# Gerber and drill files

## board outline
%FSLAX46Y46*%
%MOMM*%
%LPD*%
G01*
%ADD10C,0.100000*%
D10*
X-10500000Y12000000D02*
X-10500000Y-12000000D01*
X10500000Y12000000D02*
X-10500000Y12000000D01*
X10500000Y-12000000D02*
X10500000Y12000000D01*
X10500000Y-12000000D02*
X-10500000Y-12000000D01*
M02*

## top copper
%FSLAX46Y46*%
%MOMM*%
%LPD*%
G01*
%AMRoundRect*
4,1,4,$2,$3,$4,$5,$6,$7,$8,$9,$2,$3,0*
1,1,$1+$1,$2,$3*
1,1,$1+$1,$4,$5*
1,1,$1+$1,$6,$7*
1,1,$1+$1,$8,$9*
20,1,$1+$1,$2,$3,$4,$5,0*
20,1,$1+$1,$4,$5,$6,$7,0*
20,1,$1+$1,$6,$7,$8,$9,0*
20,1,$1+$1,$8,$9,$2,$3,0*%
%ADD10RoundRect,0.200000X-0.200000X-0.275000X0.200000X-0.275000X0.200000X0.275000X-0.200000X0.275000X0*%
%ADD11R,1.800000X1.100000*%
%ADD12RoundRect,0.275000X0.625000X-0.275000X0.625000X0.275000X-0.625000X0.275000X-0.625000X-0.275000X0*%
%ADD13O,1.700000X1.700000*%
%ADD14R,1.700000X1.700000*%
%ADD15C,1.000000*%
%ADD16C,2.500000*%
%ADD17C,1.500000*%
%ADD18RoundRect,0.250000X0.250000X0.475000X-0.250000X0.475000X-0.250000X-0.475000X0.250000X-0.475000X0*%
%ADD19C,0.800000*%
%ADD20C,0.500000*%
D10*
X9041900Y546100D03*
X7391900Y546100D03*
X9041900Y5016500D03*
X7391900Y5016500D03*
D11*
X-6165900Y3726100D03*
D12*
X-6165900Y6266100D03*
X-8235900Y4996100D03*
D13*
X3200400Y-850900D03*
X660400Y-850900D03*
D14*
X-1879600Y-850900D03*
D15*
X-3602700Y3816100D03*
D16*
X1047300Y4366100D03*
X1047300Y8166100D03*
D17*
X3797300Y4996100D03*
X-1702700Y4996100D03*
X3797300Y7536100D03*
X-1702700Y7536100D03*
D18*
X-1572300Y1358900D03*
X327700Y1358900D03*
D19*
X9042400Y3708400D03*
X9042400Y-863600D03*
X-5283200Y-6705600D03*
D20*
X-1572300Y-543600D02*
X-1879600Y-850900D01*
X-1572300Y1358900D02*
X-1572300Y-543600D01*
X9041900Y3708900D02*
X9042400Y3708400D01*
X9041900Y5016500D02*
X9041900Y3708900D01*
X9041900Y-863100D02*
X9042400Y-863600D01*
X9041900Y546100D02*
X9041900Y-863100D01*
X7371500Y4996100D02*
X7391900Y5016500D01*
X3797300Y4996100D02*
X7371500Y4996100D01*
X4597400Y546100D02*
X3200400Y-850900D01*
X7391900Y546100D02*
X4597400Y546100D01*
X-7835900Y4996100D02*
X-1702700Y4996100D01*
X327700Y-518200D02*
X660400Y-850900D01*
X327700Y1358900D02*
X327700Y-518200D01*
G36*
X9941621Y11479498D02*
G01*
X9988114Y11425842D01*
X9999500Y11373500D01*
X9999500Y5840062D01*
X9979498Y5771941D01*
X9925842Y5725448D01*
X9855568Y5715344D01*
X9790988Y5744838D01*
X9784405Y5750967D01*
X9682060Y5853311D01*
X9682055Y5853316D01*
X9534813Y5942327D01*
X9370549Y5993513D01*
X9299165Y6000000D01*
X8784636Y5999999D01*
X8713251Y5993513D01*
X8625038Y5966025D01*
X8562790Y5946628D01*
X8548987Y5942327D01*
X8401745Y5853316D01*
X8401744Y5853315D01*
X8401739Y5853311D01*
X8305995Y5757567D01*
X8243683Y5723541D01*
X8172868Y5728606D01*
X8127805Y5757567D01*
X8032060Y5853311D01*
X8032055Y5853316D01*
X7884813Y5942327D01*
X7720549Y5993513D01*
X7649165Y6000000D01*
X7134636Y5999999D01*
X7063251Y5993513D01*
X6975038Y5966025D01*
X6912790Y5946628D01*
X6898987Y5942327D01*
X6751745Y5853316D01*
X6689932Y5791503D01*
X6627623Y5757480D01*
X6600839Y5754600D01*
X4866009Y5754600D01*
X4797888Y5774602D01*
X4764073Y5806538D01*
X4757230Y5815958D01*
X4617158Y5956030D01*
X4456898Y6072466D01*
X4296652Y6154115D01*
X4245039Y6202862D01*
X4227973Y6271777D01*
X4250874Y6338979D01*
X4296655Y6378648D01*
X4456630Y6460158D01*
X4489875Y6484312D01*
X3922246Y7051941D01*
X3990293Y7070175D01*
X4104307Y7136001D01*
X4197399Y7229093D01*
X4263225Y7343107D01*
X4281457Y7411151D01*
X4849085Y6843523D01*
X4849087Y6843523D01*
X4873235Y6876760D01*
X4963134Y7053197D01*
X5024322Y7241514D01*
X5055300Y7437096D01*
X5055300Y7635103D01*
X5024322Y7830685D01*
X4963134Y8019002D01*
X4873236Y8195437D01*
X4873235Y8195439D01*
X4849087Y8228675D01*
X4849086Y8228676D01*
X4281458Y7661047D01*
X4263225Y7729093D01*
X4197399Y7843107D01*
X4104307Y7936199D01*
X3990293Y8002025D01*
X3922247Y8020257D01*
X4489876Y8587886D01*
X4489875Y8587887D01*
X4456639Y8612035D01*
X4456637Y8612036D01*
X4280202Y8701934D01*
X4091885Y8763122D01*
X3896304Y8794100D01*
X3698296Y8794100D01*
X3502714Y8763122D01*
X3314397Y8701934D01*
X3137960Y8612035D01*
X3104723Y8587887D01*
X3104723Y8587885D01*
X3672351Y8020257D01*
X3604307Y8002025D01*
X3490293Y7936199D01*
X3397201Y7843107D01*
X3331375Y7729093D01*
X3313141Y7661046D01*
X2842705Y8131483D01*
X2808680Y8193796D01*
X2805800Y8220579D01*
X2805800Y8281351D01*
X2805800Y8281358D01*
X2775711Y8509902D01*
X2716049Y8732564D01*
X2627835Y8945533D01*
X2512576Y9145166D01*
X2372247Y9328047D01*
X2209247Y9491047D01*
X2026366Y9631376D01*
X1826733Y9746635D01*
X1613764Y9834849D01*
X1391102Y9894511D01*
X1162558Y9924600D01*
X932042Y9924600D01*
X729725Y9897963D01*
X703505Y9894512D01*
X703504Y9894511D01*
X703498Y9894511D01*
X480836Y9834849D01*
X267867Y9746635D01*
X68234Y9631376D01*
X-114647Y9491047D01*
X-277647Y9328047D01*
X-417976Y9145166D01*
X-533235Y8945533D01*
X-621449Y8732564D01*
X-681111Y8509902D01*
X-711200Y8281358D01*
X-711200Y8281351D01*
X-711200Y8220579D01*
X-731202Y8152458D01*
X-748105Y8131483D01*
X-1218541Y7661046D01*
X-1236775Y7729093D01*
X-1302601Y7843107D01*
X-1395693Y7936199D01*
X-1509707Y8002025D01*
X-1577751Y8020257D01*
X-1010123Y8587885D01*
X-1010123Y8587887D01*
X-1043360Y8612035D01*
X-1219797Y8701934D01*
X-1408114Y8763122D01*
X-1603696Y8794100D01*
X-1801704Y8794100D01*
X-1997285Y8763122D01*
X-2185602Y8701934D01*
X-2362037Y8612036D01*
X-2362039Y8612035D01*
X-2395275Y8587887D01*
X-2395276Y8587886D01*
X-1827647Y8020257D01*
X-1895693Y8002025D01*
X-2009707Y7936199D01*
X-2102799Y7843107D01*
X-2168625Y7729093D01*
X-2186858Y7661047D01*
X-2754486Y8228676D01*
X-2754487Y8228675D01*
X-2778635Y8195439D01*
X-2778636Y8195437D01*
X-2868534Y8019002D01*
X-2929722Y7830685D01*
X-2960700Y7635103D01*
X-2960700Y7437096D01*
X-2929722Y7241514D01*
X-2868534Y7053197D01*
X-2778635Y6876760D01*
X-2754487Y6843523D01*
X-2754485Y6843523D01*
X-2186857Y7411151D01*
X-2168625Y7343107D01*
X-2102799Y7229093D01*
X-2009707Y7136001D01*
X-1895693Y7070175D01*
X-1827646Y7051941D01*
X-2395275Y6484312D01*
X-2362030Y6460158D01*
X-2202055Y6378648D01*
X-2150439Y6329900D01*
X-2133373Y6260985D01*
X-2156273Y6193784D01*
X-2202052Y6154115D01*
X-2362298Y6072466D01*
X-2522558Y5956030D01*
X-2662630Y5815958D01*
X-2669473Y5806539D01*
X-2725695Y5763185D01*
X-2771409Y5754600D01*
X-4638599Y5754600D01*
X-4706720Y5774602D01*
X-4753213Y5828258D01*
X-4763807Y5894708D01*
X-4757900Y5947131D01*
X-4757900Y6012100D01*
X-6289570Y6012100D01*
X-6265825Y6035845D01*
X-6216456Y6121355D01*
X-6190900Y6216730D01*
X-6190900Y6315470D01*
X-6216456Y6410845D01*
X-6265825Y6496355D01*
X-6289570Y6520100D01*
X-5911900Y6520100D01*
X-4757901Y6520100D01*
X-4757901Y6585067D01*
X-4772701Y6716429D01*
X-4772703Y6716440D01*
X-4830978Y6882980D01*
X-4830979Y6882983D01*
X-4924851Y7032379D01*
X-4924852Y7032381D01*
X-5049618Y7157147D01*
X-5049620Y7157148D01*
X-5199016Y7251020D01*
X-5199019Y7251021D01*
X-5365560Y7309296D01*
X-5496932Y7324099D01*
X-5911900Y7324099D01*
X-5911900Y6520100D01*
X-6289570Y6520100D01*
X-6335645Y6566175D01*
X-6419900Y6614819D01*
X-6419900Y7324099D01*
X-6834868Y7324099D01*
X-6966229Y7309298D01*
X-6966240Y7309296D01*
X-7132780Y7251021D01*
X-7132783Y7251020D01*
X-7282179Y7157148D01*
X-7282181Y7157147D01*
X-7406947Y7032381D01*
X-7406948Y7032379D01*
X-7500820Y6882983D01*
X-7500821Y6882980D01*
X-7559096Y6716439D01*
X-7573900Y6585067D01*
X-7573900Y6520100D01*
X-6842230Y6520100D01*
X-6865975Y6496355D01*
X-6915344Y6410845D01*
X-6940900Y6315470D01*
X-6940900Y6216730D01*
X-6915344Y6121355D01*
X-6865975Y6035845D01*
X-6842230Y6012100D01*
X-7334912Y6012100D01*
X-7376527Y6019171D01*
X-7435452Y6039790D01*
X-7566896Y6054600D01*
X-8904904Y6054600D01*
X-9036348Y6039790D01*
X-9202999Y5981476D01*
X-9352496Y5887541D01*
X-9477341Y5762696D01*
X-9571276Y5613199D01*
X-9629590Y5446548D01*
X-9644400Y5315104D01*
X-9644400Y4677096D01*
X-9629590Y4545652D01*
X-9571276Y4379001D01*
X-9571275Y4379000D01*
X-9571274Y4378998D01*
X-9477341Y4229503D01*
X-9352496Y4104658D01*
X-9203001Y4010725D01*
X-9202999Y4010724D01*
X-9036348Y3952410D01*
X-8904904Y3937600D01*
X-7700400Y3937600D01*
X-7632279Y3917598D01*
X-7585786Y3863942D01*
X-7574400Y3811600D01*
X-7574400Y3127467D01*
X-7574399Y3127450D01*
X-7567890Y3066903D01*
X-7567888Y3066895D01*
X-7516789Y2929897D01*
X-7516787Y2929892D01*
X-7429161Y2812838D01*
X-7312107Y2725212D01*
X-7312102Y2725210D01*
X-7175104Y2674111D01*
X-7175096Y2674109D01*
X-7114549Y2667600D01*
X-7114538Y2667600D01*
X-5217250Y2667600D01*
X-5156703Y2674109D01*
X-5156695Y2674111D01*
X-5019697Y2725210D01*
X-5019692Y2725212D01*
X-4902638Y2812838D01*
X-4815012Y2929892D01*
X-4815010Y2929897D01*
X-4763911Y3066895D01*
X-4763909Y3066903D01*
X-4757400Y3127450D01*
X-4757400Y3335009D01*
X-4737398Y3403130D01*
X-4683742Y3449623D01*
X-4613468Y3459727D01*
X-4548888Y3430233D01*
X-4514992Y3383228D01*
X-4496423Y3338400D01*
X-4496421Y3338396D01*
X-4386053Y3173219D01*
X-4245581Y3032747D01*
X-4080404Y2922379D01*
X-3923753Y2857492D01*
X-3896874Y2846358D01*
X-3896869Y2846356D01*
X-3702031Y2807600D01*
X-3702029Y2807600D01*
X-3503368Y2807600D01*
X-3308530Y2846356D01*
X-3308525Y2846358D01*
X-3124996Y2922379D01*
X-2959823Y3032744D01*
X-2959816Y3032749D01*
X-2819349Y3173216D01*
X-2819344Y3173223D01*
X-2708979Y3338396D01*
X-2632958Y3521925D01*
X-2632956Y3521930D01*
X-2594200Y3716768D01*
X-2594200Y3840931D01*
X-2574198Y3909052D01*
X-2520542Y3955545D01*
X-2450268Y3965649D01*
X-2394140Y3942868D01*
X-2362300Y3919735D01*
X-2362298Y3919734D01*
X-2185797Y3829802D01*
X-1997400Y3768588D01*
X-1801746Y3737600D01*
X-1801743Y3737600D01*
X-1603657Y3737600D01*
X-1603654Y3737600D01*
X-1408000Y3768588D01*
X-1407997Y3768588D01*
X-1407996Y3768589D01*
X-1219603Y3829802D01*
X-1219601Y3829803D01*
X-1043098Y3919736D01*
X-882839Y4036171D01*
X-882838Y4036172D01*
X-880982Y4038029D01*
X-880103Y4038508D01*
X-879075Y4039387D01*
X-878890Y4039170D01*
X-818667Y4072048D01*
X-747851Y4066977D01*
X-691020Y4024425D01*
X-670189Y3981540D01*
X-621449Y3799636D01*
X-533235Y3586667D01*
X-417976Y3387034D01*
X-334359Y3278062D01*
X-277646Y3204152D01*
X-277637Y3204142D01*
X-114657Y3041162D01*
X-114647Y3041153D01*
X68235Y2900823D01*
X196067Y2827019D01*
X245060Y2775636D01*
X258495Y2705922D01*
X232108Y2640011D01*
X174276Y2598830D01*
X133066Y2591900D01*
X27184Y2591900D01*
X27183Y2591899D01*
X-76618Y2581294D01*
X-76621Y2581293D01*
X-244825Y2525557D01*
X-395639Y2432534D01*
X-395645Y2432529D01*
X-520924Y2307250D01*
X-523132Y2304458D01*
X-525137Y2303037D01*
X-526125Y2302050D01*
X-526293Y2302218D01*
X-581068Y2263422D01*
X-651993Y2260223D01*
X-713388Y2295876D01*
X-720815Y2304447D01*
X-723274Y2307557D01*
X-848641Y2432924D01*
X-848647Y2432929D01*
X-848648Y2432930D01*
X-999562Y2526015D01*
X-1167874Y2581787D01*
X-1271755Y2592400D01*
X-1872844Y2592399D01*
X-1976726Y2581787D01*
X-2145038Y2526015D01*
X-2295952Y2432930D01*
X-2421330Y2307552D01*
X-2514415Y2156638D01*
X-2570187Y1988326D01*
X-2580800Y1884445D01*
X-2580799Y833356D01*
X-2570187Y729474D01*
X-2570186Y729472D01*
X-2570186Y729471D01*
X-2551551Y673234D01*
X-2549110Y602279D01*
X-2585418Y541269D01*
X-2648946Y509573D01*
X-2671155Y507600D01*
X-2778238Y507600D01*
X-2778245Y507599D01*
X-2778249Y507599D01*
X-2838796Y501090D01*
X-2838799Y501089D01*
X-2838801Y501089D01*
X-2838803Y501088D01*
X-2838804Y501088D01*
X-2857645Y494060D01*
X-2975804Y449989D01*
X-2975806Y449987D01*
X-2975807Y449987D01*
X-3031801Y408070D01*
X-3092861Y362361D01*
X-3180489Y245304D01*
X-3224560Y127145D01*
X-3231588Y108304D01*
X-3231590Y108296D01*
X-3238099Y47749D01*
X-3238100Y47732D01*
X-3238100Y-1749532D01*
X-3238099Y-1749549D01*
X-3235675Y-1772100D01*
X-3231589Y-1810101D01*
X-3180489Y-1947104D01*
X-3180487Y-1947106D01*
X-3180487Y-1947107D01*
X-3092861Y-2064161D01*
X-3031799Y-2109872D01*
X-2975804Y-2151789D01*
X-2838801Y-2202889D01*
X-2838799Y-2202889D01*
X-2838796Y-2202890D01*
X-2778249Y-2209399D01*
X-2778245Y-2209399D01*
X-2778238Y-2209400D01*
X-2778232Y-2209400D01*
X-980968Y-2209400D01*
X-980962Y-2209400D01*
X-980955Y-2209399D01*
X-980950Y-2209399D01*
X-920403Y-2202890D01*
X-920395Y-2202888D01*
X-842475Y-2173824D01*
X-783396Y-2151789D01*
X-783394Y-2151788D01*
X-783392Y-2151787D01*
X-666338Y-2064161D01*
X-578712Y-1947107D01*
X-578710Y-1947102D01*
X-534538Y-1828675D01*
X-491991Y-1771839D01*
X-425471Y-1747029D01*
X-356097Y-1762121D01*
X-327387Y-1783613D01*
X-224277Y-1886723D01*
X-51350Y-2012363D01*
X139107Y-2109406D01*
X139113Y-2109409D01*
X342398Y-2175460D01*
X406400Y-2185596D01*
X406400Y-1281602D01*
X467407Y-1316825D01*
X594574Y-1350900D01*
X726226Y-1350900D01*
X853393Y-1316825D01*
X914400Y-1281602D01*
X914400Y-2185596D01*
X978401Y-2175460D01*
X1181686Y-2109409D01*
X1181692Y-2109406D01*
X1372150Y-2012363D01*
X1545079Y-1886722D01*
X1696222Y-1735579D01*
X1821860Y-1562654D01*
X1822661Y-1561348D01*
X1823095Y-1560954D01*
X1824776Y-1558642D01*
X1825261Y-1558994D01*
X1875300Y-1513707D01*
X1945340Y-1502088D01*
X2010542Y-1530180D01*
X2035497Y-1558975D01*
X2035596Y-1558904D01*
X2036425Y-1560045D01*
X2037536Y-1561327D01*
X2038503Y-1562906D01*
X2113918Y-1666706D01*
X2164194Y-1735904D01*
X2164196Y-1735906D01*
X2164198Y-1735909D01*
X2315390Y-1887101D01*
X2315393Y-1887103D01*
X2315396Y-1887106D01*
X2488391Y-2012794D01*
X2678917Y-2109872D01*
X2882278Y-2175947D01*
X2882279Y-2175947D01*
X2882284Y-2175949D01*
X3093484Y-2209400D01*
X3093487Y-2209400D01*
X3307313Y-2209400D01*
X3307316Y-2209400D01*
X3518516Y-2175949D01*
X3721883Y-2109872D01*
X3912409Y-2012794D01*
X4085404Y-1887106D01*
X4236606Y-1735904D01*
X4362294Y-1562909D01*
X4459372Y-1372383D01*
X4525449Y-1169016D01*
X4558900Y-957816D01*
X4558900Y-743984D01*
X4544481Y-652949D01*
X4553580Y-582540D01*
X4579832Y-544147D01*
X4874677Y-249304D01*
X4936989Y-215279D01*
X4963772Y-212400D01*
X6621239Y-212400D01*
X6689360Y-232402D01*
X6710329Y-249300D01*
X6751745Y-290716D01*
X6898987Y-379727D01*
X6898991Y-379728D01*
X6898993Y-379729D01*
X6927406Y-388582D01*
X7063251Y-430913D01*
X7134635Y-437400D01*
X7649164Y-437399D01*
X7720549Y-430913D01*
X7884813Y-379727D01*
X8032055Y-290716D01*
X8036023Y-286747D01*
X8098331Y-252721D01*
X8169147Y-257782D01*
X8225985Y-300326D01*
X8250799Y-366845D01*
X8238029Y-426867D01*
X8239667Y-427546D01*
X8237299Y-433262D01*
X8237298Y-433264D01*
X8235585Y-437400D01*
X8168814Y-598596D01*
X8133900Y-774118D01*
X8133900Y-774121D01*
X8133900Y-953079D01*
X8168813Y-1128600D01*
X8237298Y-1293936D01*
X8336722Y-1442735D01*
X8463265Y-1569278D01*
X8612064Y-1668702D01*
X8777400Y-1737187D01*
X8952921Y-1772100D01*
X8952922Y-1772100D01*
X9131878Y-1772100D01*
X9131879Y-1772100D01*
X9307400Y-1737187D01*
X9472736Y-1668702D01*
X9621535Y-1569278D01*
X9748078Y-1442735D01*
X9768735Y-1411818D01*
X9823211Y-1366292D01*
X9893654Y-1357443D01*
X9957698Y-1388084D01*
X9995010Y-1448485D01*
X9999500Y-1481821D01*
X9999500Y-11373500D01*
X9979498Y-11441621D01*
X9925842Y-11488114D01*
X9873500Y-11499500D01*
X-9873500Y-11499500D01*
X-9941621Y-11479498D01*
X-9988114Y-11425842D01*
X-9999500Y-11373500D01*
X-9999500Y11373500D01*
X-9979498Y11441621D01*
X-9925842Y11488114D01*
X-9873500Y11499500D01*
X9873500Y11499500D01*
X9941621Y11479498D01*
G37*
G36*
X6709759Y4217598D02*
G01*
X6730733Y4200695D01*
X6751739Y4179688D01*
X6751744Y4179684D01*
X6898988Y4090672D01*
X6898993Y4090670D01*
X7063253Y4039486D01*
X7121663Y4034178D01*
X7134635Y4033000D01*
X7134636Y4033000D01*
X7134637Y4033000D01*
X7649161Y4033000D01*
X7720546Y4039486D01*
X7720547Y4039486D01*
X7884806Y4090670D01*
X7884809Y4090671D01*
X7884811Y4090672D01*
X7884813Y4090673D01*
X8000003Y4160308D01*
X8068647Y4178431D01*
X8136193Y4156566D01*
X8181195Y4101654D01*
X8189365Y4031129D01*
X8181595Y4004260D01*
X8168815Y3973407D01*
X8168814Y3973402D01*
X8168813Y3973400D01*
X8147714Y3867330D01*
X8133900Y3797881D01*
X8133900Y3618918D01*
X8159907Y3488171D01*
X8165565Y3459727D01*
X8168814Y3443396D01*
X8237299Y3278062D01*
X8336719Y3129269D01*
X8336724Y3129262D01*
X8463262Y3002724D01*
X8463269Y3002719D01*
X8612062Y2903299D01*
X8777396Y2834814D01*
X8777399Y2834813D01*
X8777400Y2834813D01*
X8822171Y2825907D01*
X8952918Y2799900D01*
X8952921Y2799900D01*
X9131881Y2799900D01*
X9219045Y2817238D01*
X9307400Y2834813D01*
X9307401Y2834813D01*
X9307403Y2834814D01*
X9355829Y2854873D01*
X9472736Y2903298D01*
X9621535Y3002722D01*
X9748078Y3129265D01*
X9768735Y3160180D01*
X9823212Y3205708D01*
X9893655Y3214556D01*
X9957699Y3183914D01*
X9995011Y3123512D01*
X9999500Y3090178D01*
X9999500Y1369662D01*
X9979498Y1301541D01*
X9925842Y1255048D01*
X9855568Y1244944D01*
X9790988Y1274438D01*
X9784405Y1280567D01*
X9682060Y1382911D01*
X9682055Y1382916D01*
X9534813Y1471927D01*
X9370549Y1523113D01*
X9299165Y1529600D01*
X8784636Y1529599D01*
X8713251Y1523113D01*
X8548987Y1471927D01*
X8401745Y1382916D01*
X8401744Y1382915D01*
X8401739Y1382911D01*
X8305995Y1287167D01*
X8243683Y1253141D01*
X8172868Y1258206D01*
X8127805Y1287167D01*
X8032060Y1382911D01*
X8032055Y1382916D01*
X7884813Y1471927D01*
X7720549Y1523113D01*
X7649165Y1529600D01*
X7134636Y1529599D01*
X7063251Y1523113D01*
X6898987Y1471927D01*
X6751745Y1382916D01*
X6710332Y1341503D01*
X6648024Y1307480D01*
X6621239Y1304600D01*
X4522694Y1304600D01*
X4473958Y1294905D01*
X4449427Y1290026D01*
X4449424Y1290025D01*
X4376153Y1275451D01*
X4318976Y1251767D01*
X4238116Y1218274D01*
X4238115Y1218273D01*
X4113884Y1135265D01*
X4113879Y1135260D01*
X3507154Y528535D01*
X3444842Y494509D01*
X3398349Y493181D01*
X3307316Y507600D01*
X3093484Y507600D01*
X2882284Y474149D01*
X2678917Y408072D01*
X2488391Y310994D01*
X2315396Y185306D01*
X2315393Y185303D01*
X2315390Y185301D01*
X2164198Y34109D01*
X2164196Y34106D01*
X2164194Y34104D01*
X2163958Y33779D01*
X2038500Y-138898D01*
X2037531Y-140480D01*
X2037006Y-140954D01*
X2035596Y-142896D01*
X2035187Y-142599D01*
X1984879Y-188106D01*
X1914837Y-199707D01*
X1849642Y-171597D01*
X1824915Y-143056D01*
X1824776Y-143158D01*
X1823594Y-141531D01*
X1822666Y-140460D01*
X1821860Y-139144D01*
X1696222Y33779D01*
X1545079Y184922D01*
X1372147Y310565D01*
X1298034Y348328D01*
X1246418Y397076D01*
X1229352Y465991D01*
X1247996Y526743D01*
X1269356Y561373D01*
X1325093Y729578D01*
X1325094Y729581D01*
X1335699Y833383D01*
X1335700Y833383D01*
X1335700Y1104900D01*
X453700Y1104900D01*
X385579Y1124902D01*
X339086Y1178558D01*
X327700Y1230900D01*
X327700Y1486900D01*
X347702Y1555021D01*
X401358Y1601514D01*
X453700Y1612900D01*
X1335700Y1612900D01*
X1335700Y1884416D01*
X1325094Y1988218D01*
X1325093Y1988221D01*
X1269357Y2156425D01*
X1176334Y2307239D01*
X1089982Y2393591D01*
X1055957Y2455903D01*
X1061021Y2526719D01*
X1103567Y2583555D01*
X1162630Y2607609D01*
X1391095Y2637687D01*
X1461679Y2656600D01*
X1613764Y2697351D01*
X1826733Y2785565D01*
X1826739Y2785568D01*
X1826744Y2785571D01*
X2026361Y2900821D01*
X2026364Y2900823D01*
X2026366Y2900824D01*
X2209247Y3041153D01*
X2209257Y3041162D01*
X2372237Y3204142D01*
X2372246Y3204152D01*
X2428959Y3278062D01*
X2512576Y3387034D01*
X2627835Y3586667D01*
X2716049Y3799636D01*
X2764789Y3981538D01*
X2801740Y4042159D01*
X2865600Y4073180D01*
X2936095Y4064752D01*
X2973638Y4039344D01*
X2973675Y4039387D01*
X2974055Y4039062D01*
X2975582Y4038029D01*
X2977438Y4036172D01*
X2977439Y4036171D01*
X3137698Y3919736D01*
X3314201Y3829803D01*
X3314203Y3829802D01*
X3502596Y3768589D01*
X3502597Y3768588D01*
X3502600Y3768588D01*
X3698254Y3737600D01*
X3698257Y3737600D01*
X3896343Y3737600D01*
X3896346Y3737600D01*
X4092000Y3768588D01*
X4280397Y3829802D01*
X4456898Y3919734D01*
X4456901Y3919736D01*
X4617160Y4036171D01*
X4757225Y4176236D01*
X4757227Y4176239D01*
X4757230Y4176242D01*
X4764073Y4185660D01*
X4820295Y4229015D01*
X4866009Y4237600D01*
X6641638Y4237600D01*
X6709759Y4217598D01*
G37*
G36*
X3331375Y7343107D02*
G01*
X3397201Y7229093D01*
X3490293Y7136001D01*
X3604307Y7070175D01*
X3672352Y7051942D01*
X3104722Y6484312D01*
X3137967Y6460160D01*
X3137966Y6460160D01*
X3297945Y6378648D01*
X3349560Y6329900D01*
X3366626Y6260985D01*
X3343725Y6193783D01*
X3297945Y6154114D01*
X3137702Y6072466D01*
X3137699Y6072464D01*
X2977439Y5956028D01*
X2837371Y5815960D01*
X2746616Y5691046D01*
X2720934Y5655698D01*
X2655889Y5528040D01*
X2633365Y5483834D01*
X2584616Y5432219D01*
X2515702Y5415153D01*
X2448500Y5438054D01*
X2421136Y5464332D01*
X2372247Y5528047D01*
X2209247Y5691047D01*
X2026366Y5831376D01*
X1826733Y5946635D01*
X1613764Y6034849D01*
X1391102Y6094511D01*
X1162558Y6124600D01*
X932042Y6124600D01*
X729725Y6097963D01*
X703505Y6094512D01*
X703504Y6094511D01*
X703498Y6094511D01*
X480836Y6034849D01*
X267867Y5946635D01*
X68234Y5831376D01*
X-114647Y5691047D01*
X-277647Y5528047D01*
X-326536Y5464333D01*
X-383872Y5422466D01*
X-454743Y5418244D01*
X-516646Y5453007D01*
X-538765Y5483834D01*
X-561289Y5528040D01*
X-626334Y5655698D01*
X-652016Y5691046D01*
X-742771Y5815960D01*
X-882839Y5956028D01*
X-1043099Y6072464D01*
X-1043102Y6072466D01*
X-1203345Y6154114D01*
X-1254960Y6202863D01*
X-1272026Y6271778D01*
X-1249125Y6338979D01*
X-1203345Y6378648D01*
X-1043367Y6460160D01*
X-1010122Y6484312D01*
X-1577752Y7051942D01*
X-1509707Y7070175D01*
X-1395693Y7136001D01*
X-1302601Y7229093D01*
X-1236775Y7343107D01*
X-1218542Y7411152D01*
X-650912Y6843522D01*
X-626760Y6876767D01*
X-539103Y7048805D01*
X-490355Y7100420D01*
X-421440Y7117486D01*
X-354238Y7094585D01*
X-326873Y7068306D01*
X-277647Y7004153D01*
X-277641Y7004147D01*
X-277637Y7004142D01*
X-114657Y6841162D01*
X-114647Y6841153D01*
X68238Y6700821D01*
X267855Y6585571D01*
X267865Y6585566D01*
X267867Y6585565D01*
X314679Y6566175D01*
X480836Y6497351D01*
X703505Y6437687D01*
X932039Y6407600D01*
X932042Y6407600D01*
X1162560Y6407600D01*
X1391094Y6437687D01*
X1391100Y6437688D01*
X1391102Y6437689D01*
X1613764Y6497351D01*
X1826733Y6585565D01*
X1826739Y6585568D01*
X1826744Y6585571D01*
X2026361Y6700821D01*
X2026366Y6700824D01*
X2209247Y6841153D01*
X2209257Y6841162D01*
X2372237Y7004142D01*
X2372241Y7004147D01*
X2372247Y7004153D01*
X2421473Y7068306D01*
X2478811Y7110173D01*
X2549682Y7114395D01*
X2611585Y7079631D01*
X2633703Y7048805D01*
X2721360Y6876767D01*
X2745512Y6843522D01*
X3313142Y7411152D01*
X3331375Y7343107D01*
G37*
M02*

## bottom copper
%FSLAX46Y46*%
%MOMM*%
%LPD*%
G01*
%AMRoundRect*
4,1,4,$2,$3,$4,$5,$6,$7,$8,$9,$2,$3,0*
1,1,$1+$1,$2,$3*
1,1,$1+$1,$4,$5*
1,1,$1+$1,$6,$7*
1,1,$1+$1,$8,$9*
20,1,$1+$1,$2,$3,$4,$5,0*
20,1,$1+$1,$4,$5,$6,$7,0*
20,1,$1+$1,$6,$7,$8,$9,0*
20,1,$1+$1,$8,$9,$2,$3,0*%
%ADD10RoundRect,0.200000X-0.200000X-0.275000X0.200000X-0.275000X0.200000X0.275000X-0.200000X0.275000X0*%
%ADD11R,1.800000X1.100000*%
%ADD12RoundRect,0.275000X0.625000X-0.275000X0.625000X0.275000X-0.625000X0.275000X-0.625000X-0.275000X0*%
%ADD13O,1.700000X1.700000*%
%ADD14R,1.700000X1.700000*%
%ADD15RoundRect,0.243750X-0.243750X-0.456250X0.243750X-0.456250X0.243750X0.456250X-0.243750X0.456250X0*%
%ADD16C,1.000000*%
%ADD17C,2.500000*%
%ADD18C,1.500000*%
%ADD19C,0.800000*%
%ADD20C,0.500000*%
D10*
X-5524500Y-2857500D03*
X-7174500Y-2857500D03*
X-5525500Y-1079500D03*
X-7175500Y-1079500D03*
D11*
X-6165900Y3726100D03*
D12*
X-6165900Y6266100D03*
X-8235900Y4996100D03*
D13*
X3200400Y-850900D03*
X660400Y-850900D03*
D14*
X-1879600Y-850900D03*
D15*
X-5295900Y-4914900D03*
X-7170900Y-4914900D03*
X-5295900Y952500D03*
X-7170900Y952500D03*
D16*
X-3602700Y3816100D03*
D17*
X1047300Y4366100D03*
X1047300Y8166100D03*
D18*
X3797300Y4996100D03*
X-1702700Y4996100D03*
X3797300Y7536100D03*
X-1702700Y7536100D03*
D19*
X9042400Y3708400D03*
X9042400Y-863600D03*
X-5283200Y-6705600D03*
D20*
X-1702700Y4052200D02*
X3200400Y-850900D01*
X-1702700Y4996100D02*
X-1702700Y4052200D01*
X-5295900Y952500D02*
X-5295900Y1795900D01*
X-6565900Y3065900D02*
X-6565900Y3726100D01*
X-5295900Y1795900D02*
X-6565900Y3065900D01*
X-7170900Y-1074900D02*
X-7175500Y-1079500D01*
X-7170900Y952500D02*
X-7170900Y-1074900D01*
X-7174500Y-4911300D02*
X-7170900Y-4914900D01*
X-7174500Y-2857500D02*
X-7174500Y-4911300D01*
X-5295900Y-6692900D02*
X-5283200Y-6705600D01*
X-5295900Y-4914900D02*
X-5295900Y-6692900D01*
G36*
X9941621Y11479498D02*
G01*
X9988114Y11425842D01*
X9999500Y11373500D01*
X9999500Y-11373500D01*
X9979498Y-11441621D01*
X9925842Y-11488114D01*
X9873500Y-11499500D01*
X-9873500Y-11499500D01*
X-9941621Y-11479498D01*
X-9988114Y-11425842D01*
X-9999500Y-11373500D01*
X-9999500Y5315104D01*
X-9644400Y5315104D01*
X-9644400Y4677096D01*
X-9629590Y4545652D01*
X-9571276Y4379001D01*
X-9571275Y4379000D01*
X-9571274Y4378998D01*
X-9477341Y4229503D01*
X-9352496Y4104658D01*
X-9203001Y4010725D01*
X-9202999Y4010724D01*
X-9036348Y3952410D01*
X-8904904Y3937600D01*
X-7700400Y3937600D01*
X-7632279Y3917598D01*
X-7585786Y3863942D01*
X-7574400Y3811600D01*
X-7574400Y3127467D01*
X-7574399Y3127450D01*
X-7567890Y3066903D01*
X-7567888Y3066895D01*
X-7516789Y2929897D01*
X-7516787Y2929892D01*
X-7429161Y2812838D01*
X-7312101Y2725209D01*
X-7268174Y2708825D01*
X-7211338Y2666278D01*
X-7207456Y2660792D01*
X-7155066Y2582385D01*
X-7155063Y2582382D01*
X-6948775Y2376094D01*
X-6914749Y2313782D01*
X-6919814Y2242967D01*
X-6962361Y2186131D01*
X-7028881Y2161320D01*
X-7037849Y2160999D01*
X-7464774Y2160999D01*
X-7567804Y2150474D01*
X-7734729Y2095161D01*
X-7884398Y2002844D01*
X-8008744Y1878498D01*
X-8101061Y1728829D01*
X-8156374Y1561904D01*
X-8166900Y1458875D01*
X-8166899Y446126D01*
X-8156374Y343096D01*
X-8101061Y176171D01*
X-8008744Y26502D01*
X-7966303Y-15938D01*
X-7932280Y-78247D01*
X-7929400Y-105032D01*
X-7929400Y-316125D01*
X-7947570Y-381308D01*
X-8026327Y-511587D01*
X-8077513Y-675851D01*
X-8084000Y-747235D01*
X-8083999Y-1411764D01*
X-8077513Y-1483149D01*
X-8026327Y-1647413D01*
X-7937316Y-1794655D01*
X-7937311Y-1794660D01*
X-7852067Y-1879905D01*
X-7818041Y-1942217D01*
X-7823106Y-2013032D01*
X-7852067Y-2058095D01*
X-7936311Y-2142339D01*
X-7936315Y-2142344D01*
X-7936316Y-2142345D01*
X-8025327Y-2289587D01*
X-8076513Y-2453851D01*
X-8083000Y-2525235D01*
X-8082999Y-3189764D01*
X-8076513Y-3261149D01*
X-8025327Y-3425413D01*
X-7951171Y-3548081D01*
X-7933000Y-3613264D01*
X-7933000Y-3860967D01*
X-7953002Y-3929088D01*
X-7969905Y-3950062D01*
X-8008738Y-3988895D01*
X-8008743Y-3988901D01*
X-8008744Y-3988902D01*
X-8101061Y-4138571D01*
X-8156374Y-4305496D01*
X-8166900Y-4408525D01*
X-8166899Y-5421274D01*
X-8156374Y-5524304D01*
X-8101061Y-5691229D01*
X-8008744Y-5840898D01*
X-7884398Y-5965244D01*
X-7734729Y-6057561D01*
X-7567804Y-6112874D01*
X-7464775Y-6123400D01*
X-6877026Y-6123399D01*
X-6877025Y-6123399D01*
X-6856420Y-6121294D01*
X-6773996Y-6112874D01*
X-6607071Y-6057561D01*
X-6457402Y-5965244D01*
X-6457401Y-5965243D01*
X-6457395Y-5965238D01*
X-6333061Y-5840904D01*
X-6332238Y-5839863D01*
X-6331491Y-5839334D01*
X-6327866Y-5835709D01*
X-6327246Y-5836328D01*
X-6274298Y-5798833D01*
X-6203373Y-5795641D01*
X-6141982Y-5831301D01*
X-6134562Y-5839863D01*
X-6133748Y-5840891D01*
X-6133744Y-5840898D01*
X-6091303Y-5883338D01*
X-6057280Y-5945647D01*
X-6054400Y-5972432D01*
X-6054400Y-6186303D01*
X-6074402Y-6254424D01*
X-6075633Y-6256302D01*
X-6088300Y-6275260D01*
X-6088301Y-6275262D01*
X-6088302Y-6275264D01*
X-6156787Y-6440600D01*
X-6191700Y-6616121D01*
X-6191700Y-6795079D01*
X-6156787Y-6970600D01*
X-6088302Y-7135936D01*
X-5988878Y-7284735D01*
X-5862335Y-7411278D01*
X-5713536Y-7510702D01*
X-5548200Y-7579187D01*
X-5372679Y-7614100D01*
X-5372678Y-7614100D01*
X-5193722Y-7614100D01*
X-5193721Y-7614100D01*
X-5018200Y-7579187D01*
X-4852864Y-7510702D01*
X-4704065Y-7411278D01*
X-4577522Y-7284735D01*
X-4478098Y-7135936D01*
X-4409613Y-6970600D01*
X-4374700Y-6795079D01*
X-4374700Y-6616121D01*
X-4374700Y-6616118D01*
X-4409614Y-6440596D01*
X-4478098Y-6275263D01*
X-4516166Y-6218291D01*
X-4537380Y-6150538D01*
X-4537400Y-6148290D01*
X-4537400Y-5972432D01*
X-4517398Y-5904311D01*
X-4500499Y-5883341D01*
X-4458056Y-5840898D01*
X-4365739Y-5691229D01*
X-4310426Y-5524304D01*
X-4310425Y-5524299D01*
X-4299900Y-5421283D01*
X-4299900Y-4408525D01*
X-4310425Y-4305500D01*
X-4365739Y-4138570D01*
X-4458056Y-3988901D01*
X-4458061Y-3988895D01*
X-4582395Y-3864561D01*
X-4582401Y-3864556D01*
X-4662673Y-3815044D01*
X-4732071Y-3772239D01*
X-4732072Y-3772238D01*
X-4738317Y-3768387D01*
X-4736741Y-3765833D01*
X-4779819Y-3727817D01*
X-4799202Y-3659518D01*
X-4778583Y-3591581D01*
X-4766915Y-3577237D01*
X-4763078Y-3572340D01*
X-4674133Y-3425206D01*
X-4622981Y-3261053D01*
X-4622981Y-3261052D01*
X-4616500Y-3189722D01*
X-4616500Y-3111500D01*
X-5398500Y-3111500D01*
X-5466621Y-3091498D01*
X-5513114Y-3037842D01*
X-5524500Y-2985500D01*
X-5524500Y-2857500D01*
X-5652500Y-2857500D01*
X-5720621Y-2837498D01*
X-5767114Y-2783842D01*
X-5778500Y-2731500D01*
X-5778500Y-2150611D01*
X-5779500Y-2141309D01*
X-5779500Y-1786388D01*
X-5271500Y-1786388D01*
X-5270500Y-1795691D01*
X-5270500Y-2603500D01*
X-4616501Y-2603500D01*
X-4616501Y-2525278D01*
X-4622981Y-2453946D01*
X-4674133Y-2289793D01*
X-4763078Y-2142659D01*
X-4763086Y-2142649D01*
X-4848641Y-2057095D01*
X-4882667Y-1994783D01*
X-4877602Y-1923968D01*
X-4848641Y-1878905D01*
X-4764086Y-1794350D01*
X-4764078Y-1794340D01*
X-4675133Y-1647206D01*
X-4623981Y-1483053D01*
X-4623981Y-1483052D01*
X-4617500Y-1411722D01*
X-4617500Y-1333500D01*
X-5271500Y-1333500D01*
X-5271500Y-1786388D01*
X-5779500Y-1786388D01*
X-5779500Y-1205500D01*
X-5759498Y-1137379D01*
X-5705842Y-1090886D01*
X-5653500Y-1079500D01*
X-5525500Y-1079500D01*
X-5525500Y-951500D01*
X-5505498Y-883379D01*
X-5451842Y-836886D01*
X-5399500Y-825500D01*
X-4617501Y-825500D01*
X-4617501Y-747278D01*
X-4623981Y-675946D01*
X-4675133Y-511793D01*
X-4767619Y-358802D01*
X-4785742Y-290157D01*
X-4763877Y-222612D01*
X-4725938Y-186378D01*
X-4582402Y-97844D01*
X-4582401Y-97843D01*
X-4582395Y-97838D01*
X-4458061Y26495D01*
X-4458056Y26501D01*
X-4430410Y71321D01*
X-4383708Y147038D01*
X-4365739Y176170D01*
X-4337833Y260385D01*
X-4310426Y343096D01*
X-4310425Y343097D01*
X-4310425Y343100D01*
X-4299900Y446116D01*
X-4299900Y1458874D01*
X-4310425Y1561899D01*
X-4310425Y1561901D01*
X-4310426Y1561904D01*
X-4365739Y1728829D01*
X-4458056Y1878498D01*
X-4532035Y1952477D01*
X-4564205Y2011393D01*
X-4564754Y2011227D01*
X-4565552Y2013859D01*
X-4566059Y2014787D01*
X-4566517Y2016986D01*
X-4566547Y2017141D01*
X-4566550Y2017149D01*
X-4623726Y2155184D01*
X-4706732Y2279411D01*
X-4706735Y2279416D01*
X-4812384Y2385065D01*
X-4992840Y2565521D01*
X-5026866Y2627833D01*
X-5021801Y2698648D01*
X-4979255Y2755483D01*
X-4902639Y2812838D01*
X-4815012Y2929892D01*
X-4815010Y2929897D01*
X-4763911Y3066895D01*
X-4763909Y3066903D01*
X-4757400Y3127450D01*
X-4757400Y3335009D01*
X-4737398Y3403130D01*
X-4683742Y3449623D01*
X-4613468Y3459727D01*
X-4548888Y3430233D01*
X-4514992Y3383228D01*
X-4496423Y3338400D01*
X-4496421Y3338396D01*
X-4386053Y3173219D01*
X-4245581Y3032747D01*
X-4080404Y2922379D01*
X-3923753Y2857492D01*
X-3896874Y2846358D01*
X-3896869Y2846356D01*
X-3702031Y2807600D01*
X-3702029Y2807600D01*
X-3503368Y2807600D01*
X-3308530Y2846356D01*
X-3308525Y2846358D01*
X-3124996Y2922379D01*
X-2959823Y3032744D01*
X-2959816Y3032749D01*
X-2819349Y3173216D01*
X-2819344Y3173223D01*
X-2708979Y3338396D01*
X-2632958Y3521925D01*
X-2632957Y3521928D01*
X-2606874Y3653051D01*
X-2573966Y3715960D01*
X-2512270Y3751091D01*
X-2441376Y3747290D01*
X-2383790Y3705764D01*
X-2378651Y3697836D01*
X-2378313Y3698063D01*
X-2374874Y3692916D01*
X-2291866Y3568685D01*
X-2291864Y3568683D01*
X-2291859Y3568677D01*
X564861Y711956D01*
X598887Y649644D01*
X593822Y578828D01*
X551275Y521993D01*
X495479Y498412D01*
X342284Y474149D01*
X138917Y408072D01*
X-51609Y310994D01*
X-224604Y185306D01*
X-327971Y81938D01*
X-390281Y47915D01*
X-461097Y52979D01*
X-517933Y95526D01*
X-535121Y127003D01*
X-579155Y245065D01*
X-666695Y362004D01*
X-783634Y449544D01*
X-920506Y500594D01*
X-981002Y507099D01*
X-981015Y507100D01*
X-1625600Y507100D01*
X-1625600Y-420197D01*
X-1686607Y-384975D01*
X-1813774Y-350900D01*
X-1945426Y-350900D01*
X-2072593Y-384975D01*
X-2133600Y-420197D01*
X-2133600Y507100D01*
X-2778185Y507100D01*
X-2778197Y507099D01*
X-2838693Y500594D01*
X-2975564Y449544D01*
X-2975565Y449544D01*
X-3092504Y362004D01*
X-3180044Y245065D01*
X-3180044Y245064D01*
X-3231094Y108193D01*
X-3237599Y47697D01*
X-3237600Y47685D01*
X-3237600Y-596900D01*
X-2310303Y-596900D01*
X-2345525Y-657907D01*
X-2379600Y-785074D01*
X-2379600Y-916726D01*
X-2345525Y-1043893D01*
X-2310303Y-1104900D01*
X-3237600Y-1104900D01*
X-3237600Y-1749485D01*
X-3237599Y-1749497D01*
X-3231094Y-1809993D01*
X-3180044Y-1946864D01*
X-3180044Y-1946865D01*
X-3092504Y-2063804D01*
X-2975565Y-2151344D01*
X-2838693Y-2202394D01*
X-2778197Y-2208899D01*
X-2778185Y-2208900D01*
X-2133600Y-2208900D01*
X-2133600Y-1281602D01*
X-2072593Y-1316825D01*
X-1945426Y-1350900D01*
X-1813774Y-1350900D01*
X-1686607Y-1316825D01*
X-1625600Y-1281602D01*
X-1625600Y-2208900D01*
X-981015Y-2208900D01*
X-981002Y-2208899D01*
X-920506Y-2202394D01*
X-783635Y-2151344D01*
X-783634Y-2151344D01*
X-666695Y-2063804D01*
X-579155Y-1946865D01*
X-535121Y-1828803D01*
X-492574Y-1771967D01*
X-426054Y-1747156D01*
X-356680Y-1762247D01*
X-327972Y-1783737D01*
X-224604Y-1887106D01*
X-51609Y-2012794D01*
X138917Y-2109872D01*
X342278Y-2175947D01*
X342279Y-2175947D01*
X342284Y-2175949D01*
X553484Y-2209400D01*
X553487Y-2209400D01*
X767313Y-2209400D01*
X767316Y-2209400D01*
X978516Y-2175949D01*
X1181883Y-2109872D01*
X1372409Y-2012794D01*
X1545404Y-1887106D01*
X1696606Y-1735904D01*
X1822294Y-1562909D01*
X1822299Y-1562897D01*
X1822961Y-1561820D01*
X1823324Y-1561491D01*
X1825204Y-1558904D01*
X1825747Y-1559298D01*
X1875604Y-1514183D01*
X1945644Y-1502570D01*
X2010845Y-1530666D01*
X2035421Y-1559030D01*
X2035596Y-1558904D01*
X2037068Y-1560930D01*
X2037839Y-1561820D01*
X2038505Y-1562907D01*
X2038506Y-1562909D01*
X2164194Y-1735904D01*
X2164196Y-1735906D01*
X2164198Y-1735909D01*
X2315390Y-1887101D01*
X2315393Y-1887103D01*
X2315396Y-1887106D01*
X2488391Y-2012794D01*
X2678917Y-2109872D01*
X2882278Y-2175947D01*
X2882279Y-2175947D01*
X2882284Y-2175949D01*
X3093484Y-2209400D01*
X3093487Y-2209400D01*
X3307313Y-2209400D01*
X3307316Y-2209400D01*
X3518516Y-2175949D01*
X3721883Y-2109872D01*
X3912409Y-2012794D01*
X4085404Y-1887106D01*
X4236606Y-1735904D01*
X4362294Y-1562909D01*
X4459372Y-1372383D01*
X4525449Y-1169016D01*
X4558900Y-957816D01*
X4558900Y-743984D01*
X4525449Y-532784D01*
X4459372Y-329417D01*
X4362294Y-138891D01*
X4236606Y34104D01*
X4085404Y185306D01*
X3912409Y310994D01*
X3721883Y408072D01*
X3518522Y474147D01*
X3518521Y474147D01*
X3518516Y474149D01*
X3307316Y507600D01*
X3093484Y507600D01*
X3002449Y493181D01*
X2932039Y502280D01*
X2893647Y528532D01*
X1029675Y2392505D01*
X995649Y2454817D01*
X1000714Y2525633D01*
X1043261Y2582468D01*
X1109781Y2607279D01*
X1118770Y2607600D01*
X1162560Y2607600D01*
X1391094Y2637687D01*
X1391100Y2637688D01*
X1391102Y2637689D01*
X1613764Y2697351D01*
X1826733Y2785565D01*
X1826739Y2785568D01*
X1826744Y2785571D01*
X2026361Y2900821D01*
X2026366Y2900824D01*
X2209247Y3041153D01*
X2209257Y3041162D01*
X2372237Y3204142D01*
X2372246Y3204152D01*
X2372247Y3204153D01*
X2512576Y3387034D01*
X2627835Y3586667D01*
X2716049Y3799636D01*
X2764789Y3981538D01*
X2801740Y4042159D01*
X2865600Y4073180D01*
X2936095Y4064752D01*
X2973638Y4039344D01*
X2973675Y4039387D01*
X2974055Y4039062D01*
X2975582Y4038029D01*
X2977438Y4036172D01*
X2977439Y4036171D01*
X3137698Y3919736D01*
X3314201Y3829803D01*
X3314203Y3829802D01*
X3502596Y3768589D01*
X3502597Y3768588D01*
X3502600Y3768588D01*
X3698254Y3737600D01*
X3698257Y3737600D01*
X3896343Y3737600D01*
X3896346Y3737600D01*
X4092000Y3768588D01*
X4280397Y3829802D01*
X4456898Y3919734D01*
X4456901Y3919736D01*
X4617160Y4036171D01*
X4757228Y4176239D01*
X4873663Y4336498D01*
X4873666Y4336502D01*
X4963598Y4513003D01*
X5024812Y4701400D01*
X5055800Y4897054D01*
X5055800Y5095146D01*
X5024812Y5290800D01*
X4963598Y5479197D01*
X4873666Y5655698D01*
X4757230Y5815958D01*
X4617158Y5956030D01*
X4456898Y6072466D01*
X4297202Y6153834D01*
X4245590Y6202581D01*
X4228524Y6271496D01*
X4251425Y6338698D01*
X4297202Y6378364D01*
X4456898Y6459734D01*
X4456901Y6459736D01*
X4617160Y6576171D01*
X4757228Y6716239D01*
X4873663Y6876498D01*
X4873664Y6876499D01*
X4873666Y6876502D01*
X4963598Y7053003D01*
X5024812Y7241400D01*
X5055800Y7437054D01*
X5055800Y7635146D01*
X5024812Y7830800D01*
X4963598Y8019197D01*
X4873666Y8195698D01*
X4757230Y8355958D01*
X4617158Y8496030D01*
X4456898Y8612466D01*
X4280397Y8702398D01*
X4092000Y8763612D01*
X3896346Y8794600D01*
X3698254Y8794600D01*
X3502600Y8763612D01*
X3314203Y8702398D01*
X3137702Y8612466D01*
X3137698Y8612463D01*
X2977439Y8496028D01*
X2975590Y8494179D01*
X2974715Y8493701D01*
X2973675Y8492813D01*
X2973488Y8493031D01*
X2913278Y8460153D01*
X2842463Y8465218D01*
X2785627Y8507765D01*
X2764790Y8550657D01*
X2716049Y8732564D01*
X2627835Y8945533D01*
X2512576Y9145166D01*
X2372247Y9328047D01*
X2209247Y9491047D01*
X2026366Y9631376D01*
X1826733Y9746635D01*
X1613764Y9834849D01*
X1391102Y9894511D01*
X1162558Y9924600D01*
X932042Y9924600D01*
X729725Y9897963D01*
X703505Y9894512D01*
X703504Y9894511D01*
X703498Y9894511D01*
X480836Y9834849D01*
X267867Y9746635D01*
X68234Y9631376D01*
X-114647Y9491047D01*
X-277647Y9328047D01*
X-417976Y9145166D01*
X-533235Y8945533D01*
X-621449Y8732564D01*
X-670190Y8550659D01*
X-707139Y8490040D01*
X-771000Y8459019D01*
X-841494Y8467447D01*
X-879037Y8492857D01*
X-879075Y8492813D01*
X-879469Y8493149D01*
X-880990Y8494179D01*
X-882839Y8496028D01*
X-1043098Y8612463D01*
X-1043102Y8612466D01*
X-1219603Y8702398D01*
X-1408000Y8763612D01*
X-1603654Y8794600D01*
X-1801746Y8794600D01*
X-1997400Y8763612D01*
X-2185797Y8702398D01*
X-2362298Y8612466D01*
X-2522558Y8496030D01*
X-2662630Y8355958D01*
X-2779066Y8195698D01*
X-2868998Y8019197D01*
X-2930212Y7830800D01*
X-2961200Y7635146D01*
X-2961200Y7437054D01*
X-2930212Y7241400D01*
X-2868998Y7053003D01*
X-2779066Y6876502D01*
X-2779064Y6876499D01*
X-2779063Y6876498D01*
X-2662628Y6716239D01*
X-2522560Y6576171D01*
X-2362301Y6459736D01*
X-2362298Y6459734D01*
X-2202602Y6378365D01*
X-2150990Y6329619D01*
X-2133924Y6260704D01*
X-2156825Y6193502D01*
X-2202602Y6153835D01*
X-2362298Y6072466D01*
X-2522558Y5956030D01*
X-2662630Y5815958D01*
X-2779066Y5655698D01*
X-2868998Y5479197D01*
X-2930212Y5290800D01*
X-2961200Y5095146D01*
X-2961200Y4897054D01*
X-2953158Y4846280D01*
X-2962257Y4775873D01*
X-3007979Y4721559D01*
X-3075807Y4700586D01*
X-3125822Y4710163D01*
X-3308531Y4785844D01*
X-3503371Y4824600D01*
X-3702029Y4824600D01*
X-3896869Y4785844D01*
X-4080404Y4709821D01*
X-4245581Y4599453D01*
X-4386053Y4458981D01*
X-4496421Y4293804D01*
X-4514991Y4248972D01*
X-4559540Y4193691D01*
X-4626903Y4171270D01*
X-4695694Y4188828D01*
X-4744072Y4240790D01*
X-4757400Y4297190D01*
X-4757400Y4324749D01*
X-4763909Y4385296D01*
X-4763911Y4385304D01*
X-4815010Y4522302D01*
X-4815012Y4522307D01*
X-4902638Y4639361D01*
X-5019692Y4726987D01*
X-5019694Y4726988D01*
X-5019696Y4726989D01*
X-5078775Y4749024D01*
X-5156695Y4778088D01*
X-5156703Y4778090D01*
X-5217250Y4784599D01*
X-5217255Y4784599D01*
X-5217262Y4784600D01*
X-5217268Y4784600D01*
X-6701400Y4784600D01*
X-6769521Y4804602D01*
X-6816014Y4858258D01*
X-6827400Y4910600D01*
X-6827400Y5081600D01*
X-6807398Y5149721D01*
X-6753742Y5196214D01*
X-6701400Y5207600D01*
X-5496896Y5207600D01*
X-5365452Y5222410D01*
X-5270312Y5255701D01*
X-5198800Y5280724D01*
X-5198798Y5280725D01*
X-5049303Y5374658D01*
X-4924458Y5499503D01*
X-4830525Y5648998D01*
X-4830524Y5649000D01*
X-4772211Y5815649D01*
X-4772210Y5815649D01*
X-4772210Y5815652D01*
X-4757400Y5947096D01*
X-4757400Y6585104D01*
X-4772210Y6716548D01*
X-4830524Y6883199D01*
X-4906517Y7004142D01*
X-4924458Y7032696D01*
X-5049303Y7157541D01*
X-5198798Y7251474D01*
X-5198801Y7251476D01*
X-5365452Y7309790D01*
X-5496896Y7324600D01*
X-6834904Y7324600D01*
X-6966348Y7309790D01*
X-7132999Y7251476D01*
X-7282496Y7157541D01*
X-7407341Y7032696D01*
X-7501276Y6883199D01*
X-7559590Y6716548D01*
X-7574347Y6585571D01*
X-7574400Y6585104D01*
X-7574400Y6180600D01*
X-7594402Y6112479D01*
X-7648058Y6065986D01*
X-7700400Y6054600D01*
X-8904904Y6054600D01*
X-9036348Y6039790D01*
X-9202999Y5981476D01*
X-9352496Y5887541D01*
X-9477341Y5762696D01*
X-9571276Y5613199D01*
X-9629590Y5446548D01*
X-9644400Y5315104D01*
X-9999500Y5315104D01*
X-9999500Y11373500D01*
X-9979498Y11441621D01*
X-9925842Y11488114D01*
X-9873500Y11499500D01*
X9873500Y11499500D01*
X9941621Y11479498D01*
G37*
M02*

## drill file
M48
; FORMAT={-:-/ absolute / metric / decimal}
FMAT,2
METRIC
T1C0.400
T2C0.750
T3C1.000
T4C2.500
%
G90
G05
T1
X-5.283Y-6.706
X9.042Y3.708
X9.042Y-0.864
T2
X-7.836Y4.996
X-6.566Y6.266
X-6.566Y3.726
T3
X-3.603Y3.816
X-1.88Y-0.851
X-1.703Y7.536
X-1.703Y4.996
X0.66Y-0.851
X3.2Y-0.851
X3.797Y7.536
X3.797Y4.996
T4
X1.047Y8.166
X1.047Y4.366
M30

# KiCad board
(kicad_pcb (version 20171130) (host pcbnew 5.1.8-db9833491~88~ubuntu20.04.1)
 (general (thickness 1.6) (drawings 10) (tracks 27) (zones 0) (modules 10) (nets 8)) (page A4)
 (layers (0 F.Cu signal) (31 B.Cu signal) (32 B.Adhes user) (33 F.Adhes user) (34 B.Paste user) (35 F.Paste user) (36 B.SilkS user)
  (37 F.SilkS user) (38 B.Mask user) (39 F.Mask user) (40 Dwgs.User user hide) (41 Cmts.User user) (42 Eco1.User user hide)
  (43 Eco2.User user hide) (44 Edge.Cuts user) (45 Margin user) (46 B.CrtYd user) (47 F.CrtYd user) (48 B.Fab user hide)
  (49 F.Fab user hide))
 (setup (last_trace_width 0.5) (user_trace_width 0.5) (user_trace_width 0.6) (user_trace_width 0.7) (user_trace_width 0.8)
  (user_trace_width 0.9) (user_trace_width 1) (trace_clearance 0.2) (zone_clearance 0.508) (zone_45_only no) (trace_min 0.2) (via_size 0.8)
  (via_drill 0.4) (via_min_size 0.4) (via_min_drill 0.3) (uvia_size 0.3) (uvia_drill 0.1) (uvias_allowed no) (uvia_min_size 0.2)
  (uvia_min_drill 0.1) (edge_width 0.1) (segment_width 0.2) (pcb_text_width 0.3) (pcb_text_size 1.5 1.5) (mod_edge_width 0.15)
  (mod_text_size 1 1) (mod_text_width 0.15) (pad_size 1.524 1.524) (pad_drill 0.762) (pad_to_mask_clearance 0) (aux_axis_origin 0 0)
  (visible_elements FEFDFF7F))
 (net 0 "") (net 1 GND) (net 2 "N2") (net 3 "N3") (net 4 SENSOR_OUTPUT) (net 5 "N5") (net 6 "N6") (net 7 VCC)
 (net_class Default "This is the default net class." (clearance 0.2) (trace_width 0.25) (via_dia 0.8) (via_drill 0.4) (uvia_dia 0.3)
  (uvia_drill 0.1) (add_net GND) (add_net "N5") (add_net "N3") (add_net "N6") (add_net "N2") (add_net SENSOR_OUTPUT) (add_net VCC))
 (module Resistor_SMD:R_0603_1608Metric (layer B.Cu) (at -6.3495 2.8575)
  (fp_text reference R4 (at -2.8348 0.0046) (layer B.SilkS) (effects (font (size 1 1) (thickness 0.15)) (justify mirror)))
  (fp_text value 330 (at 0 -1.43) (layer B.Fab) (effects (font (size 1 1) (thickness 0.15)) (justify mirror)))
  (pad 2 smd roundrect (at 0.825 0) (size 0.8 0.95) (layers B.Cu B.Paste B.Mask) (roundrect_rratio 0.25) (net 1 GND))
  (pad 1 smd roundrect (at -0.825 0) (size 0.8 0.95) (layers B.Cu B.Paste B.Mask) (roundrect_rratio 0.25) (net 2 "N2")))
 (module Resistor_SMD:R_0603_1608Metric (layer B.Cu) (at -6.3505 1.0795)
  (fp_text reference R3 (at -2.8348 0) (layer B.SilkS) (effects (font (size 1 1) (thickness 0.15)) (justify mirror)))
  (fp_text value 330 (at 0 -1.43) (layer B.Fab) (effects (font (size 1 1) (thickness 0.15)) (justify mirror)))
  (pad 2 smd roundrect (at 0.825 0) (size 0.8 0.95) (layers B.Cu B.Paste B.Mask) (roundrect_rratio 0.25) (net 1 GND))
  (pad 1 smd roundrect (at -0.825 0) (size 0.8 0.95) (layers B.Cu B.Paste B.Mask) (roundrect_rratio 0.25) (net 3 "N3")))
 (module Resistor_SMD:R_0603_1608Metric (layer F.Cu) (at 8.2169 -0.5461)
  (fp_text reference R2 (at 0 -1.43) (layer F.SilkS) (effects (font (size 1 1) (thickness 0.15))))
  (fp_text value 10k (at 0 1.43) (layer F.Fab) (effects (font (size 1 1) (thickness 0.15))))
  (pad 2 smd roundrect (at 0.825 0) (size 0.8 0.95) (layers F.Cu F.Paste F.Mask) (roundrect_rratio 0.25) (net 1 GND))
  (pad 1 smd roundrect (at -0.825 0) (size 0.8 0.95) (layers F.Cu F.Paste F.Mask) (roundrect_rratio 0.25) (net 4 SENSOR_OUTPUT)))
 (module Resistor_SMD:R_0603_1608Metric (layer F.Cu) (at 8.2169 -5.0165)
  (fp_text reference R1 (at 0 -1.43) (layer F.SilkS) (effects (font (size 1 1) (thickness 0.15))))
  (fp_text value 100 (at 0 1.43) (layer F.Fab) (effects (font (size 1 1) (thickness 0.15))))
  (pad 2 smd roundrect (at 0.825 0) (size 0.8 0.95) (layers F.Cu F.Paste F.Mask) (roundrect_rratio 0.25) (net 1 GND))
  (pad 1 smd roundrect (at -0.825 0) (size 0.8 0.95) (layers F.Cu F.Paste F.Mask) (roundrect_rratio 0.25) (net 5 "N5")))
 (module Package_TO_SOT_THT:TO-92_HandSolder (layer F.Cu) (at -6.5659 -3.7261 90)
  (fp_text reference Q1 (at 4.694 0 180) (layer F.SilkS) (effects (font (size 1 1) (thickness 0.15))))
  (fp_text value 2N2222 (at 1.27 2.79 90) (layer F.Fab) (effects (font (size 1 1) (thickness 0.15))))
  (pad 1 thru_hole rect (at 0 0 90) (size 1.1 1.8) (drill 0.75 (offset 0 0.4)) (layers *.Cu *.Mask) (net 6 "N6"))
  (pad 3 thru_hole roundrect (at 2.54 0 90) (size 1.1 1.8) (drill 0.75 (offset 0 0.4)) (layers *.Cu *.Mask) (roundrect_rratio 0.25)
   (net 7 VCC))
  (pad 2 thru_hole roundrect (at 1.27 -1.27 90) (size 1.1 1.8) (drill 0.75 (offset 0 -0.4)) (layers *.Cu *.Mask) (roundrect_rratio 0.25)
   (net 4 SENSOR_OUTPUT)))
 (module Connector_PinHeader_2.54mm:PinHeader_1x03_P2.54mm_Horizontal (layer B.Cu) (at -1.8796 0.8509 270)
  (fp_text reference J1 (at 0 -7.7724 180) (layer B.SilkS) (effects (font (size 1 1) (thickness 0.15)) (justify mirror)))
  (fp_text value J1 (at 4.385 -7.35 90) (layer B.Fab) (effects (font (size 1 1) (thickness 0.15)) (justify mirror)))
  (pad 3 thru_hole oval (at 0 -5.08 270) (size 1.7 1.7) (drill 1) (layers *.Cu *.Mask) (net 4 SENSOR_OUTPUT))
  (pad 2 thru_hole oval (at 0 -2.54 270) (size 1.7 1.7) (drill 1) (layers *.Cu *.Mask) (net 7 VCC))
  (pad 1 thru_hole rect (at 0 0 270) (size 1.7 1.7) (drill 1) (layers *.Cu *.Mask) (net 1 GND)))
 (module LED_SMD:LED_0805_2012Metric (layer B.Cu) (at -6.2334 4.9149)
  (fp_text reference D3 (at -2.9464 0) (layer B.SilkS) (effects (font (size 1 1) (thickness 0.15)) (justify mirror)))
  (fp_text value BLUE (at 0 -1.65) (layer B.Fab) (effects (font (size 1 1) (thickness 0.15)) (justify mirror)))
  (pad 2 smd roundrect (at 0.9375 0) (size 0.975 1.4) (layers B.Cu B.Paste B.Mask) (roundrect_rratio 0.25) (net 7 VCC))
  (pad 1 smd roundrect (at -0.9375 0) (size 0.975 1.4) (layers B.Cu B.Paste B.Mask) (roundrect_rratio 0.25) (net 2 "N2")))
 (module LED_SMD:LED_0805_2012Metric (layer B.Cu) (at -6.2334 -0.9525)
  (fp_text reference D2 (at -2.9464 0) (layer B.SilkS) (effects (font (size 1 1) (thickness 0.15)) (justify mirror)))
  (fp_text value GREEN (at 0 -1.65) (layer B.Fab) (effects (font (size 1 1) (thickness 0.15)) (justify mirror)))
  (pad 2 smd roundrect (at 0.9375 0) (size 0.975 1.4) (layers B.Cu B.Paste B.Mask) (roundrect_rratio 0.25) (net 6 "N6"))
  (pad 1 smd roundrect (at -0.9375 0) (size 0.975 1.4) (layers B.Cu B.Paste B.Mask) (roundrect_rratio 0.25) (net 3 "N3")))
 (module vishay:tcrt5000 (layer F.Cu) (at 1.0473 -6.2661)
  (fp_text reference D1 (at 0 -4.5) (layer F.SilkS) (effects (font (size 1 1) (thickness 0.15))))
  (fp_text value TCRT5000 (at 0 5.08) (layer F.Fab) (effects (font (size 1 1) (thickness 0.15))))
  (pad 7 thru_hole circle (at -4.65 2.45) (size 1 1) (drill 1) (layers *.Cu *.Mask))
  (pad 6 thru_hole circle (at 0 1.9) (size 2.5 2.5) (drill 2.5) (layers *.Cu *.Mask))
  (pad 5 thru_hole circle (at 0 -1.9) (size 2.5 2.5) (drill 2.5) (layers *.Cu *.Mask))
  (pad 4 thru_hole circle (at 2.75 1.27) (size 1.5 1.5) (drill 1) (layers *.Cu *.Mask) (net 5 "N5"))
  (pad 3 thru_hole circle (at -2.75 1.27) (size 1.5 1.5) (drill 1) (layers *.Cu *.Mask) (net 4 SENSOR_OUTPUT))
  (pad 2 thru_hole circle (at 2.75 -1.27) (size 1.5 1.5) (drill 1) (layers *.Cu *.Mask) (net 7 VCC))
  (pad 1 thru_hole circle (at -2.75 -1.27) (size 1.5 1.5) (drill 1) (layers *.Cu *.Mask) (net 7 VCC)))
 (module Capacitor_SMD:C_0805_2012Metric (layer F.Cu) (at -0.6223 -1.3589 180)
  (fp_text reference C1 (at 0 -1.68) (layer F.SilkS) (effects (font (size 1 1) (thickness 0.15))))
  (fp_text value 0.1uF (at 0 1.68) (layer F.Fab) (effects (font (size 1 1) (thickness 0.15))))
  (pad 2 smd roundrect (at 0.95 0 180) (size 1 1.45) (layers F.Cu F.Paste F.Mask) (roundrect_rratio 0.25) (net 1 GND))
  (pad 1 smd roundrect (at -0.95 0 180) (size 1 1.45) (layers F.Cu F.Paste F.Mask) (roundrect_rratio 0.25) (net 7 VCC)))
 (gr_line (start -10.5 -12) (end -10.5 12) (layer Edge.Cuts) (width 0.1))
 (gr_line (start 10.5 -12) (end -10.5 -12) (layer Edge.Cuts) (width 0.1))
 (gr_line (start 10.5 12) (end 10.5 -12) (layer Edge.Cuts) (width 0.1))
 (gr_line (start 10.5 12) (end -10.5 12) (layer Edge.Cuts) (width 0.1))
 (segment (start -1.5723 0.5436) (end -1.8796 0.8509) (width 0.5) (layer F.Cu) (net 1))
 (segment (start -1.5723 -1.3589) (end -1.5723 0.5436) (width 0.5) (layer F.Cu) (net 1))
 (via (at 9.0424 -3.7084) (size 0.8) (drill 0.4) (layers F.Cu B.Cu) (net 1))
 (segment (start 9.0419 -3.7089) (end 9.0424 -3.7084) (width 0.5) (layer F.Cu) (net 1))
 (segment (start 9.0419 -5.0165) (end 9.0419 -3.7089) (width 0.5) (layer F.Cu) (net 1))
 (via (at 9.0424 0.8636) (size 0.8) (drill 0.4) (layers F.Cu B.Cu) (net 1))
 (segment (start 9.0419 0.8631) (end 9.0424 0.8636) (width 0.5) (layer F.Cu) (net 1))
 (segment (start 9.0419 -0.5461) (end 9.0419 0.8631) (width 0.5) (layer F.Cu) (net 1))
 (segment (start 7.3715 -4.9961) (end 7.3919 -5.0165) (width 0.5) (layer F.Cu) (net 5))
 (segment (start 3.7973 -4.9961) (end 7.3715 -4.9961) (width 0.5) (layer F.Cu) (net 5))
 (segment (start 4.5974 -0.5461) (end 3.2004 0.8509) (width 0.5) (layer F.Cu) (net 4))
 (segment (start 7.3919 -0.5461) (end 4.5974 -0.5461) (width 0.5) (layer F.Cu) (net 4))
 (segment (start -7.8359 -4.9961) (end -1.7027 -4.9961) (width 0.5) (layer F.Cu) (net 4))
 (segment (start -1.7027 -4.0522) (end 3.2004 0.8509) (width 0.5) (layer B.Cu) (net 4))
 (segment (start -1.7027 -4.9961) (end -1.7027 -4.0522) (width 0.5) (layer B.Cu) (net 4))
 (segment (start -5.2959 -0.9525) (end -5.2959 -1.7959) (width 0.5) (layer B.Cu) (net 6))
 (segment (start -6.5659 -3.0659) (end -6.5659 -3.7261) (width 0.5) (layer B.Cu) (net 6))
 (segment (start -5.2959 -1.7959) (end -6.5659 -3.0659) (width 0.5) (layer B.Cu) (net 6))
 (segment (start -7.1709 1.0749) (end -7.1755 1.0795) (width 0.5) (layer B.Cu) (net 3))
 (segment (start -7.1709 -0.9525) (end -7.1709 1.0749) (width 0.5) (layer B.Cu) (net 3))
 (segment (start -7.1745 4.9113) (end -7.1709 4.9149) (width 0.5) (layer B.Cu) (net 2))
 (segment (start -7.1745 2.8575) (end -7.1745 4.9113) (width 0.5) (layer B.Cu) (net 2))
 (segment (start 0.3277 0.5182) (end 0.6604 0.8509) (width 0.5) (layer F.Cu) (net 7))
 (segment (start 0.3277 -1.3589) (end 0.3277 0.5182) (width 0.5) (layer F.Cu) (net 7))
 (via (at -5.2832 6.7056) (size 0.8) (drill 0.4) (layers F.Cu B.Cu) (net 7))
 (segment (start -5.2959 6.6929) (end -5.2832 6.7056) (width 0.5) (layer B.Cu) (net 7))
 (segment (start -5.2959 4.9149) (end -5.2959 6.6929) (width 0.5) (layer B.Cu) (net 7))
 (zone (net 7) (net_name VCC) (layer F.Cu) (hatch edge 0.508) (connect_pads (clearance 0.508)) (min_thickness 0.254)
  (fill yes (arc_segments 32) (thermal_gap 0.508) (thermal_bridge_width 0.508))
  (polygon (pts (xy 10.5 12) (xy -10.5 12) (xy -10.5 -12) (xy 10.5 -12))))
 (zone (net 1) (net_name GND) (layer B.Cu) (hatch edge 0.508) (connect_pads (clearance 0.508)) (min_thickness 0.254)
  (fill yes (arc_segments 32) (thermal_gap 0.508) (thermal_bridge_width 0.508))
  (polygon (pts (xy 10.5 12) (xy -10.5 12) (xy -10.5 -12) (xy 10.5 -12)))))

